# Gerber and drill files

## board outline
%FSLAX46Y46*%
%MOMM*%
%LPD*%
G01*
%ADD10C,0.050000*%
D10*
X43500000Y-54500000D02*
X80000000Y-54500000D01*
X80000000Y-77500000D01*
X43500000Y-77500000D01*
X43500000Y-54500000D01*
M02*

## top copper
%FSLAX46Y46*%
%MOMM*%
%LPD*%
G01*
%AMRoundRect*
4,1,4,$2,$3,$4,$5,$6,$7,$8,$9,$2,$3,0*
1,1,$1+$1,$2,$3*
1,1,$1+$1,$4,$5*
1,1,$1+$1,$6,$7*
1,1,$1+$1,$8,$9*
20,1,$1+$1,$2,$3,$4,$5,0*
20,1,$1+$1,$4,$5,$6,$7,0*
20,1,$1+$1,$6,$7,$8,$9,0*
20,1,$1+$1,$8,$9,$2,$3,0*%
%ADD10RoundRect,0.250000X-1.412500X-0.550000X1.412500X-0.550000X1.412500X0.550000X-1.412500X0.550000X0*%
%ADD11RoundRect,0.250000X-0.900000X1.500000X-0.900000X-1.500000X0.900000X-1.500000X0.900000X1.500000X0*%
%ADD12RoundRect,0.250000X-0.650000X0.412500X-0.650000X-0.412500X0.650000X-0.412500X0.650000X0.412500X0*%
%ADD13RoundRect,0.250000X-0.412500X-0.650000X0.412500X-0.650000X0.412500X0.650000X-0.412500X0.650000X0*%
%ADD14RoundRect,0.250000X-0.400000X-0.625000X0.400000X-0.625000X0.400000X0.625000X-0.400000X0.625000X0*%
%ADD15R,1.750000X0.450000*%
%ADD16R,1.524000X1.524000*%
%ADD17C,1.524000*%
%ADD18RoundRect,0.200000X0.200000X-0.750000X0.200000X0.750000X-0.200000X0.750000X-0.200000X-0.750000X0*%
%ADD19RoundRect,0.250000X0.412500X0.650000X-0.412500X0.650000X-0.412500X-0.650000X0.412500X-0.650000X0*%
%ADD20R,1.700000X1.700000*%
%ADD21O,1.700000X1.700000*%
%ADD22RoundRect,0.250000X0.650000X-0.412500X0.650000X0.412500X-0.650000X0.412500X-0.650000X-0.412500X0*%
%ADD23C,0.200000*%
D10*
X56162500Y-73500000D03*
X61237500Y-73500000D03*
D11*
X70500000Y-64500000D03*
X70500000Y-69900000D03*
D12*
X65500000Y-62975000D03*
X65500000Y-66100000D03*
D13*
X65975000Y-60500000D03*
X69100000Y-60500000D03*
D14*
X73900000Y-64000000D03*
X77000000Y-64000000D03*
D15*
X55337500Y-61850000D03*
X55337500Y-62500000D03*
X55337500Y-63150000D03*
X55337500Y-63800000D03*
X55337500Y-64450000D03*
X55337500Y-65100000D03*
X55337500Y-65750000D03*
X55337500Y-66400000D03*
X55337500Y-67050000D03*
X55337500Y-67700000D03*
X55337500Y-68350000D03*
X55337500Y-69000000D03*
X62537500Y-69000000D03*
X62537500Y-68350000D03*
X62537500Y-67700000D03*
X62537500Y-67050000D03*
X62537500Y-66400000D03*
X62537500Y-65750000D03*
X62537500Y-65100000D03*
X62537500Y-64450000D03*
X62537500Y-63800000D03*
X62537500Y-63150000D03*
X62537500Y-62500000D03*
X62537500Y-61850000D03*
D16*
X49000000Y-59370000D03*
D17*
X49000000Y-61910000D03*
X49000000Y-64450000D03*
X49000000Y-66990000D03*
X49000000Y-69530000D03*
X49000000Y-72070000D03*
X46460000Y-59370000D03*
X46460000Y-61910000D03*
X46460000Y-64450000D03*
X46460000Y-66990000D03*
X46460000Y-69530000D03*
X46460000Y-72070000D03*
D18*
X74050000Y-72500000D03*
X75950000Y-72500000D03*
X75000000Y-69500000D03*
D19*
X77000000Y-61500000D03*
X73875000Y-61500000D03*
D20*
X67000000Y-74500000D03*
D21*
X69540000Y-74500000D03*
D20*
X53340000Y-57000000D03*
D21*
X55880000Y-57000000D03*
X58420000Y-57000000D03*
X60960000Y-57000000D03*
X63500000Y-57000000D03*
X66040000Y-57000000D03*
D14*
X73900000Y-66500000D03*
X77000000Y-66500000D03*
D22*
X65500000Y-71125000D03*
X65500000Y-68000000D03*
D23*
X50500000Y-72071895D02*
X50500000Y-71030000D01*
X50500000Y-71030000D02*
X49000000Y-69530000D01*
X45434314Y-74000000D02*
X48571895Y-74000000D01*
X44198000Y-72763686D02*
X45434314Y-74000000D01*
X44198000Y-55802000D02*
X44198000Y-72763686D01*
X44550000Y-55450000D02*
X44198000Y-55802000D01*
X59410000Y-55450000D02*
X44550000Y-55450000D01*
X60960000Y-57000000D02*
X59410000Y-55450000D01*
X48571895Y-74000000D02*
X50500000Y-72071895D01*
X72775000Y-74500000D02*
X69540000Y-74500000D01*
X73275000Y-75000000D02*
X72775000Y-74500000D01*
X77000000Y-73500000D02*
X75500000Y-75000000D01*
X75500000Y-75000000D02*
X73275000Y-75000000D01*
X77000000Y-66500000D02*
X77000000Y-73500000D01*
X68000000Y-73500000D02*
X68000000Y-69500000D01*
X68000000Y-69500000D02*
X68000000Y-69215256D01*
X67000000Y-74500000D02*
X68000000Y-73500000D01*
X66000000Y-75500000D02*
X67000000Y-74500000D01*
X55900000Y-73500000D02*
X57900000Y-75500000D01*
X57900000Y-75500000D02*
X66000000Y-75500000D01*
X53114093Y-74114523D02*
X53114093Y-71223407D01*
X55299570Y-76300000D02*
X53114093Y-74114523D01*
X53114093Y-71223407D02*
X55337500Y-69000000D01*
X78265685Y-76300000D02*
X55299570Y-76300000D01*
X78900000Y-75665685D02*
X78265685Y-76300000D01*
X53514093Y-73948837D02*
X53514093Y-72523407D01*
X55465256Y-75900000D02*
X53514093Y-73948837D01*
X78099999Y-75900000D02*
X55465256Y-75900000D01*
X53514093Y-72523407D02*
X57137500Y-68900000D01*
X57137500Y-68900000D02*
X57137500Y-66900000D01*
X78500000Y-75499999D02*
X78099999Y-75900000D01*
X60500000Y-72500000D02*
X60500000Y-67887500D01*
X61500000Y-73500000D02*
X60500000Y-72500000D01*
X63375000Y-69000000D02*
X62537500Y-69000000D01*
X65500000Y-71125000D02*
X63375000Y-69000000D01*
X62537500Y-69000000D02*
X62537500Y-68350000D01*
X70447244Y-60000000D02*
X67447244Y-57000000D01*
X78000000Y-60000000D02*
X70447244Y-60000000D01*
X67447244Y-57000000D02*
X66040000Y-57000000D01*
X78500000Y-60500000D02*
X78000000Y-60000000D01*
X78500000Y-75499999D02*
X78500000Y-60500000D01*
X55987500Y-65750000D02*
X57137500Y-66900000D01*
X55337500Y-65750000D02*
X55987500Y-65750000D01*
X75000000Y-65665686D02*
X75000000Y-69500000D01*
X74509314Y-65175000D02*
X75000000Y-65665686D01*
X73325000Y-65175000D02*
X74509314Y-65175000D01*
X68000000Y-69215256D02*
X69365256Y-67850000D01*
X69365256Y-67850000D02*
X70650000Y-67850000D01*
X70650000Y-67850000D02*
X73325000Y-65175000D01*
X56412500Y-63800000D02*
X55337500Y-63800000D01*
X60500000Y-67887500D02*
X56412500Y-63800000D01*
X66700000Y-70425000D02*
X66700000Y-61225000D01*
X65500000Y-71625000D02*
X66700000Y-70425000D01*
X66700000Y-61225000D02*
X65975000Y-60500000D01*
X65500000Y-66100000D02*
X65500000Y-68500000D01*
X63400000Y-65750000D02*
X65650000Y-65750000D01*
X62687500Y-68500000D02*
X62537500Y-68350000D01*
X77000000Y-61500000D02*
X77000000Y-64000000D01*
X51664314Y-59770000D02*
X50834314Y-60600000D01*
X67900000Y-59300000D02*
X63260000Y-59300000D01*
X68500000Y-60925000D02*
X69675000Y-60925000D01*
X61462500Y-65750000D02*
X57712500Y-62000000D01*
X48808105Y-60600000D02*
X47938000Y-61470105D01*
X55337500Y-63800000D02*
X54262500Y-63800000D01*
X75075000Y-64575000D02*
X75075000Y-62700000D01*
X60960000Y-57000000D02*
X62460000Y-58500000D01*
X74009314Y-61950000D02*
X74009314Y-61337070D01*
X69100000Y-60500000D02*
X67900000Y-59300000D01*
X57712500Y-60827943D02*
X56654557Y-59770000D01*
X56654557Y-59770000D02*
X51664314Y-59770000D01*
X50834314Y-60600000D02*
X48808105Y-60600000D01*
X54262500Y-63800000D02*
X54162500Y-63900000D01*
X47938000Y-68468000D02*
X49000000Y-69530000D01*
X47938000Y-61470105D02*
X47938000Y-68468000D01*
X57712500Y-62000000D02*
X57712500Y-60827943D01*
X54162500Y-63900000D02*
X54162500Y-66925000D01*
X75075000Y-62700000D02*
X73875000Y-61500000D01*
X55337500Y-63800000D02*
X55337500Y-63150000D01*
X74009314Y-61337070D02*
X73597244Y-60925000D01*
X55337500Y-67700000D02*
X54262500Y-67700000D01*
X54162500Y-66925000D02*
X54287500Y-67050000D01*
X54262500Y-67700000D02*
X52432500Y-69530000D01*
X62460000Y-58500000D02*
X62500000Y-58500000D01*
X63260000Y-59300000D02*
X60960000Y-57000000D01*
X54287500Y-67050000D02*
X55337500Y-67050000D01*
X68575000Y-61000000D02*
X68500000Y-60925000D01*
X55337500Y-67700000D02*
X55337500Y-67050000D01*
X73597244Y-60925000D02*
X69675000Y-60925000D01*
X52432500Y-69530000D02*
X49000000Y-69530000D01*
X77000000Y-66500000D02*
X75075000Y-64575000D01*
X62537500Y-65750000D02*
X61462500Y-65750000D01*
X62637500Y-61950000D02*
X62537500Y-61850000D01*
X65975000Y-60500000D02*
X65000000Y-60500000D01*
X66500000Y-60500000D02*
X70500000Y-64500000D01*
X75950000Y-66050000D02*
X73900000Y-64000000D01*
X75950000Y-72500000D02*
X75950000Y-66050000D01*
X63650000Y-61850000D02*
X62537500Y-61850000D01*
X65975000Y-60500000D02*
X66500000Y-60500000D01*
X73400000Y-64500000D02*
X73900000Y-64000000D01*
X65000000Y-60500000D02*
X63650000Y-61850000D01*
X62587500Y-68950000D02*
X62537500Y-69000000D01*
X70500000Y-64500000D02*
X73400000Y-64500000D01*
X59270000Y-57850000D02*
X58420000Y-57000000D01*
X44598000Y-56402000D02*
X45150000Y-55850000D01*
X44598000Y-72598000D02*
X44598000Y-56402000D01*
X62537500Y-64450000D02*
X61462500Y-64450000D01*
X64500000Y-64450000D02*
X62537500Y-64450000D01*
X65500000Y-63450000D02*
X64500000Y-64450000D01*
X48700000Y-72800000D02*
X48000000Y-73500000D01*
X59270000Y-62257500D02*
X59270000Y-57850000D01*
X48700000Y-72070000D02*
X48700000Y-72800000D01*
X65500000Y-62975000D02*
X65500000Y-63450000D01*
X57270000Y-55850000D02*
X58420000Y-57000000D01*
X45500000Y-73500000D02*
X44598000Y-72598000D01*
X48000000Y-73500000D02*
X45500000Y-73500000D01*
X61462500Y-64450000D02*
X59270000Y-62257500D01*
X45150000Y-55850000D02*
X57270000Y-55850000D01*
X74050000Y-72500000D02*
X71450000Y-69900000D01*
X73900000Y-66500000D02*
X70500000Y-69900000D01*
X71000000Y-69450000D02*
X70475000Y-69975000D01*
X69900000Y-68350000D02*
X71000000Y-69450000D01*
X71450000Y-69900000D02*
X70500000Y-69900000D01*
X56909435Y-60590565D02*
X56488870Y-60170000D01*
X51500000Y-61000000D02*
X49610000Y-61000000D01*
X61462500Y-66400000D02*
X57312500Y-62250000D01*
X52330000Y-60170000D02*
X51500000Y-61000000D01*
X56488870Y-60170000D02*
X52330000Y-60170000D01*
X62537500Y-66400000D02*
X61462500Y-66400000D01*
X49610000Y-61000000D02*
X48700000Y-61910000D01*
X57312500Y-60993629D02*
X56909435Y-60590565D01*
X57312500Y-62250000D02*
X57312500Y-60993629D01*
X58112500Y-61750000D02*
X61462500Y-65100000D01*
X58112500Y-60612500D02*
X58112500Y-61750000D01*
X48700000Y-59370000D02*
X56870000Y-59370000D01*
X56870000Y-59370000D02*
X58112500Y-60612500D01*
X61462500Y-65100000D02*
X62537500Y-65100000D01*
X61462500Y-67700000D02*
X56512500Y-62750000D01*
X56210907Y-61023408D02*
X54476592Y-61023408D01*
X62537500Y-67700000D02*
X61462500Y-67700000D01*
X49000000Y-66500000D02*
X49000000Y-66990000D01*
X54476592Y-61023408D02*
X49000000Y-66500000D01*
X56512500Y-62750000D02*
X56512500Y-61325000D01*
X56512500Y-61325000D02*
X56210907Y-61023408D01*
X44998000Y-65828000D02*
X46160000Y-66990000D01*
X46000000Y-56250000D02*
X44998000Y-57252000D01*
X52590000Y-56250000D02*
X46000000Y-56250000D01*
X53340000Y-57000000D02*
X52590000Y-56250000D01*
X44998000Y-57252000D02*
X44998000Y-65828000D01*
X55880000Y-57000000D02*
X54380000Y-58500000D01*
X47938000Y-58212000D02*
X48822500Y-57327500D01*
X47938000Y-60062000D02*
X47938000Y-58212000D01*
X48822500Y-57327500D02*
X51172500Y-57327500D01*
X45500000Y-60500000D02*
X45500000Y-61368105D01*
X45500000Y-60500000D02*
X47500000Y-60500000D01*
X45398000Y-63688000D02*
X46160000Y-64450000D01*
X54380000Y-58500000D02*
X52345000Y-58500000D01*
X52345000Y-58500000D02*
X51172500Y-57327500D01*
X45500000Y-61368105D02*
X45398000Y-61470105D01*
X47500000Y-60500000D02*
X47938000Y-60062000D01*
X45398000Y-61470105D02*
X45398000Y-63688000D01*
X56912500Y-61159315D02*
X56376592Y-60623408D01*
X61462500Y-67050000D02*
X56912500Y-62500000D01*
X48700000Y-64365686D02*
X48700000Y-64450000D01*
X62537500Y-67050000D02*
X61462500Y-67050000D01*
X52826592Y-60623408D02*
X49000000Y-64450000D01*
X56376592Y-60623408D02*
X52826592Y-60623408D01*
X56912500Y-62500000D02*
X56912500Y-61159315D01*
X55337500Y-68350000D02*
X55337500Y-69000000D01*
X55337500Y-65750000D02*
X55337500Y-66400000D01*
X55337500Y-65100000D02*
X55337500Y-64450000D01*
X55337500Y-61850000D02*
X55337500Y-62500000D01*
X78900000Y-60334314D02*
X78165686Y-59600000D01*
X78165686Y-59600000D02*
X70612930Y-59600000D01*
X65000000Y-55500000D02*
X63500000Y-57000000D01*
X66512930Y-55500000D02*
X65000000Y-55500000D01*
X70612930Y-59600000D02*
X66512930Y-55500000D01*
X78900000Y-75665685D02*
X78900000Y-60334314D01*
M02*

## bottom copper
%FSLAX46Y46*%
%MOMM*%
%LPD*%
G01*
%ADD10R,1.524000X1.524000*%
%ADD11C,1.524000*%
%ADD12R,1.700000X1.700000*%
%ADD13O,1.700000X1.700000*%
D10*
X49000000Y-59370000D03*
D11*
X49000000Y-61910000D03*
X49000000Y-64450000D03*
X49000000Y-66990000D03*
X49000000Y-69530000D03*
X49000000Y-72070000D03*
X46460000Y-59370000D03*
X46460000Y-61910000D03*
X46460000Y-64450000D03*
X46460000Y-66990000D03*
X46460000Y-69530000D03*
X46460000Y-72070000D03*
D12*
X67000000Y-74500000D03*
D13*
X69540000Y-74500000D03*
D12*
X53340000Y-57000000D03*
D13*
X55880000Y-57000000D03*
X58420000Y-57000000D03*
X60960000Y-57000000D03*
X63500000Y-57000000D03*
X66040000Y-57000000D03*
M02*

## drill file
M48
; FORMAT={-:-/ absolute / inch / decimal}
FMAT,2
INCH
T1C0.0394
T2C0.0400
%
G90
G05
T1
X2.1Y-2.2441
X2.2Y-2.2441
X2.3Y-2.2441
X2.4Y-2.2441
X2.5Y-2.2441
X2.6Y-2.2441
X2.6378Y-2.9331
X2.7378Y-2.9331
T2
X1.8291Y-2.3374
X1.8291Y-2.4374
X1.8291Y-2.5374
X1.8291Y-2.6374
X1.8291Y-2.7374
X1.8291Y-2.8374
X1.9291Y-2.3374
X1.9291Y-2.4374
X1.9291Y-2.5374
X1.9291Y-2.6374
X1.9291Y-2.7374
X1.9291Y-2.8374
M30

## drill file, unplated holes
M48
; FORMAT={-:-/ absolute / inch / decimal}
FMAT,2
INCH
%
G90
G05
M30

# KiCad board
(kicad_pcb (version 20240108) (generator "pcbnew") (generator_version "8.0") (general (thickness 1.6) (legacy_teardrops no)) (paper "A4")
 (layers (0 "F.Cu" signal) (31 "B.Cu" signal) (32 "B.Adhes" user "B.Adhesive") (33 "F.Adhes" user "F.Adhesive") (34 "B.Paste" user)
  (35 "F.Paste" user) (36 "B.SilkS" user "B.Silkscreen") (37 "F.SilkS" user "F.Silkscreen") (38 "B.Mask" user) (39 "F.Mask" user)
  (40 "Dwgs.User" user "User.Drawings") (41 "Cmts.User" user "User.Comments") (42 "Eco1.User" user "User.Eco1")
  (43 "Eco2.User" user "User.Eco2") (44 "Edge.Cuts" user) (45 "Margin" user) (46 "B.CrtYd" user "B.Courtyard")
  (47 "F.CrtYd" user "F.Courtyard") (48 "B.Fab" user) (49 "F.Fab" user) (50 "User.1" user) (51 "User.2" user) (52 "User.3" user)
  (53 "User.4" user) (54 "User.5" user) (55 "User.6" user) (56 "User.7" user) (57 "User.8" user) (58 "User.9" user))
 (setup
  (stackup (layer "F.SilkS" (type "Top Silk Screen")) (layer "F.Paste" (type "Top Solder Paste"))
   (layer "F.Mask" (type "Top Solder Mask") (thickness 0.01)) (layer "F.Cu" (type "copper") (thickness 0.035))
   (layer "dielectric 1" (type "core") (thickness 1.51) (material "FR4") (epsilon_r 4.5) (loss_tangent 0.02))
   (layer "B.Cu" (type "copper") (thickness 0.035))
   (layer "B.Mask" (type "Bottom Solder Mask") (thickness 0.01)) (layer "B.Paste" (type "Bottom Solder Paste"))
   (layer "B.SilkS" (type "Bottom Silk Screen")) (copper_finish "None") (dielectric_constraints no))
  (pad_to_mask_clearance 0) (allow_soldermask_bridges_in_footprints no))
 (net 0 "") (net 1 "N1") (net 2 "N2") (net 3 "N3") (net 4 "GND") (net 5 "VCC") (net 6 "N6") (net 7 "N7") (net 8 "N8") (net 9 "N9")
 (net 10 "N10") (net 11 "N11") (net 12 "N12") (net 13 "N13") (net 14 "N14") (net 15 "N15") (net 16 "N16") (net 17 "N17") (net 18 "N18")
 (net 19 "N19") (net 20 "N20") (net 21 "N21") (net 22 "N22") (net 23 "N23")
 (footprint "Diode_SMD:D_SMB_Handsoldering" (layer "F.Cu") (at 70.5 67.2 -90)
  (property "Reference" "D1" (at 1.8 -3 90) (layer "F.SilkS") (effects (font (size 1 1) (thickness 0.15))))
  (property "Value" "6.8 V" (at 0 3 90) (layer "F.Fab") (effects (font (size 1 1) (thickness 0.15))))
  (pad "1" smd roundrect (at -2.7 0 270) (size 3.5 2.3) (layers "F.Cu" "F.Paste" "F.Mask") (roundrect_rratio 0.1086956522) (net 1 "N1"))
  (pad "2" smd roundrect (at 2.7 0 270) (size 3.5 2.3) (layers "F.Cu" "F.Paste" "F.Mask") (roundrect_rratio 0.1086956522) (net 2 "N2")))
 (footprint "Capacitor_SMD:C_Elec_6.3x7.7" (layer "F.Cu") (at 58.7 73.5)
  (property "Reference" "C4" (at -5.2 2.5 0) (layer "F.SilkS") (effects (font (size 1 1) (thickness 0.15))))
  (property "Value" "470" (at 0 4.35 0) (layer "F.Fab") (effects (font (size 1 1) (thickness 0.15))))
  (pad "1" smd roundrect (at -2.5375 0) (size 3.325 1.6) (layers "F.Cu" "F.Paste" "F.Mask") (roundrect_rratio 0.15625) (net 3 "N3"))
  (pad "2" smd roundrect (at 2.5375 0) (size 3.325 1.6) (layers "F.Cu" "F.Paste" "F.Mask") (roundrect_rratio 0.15625) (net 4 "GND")))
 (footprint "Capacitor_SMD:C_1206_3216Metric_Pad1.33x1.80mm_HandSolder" (layer "F.Cu") (at 65.5 64.5375 -90)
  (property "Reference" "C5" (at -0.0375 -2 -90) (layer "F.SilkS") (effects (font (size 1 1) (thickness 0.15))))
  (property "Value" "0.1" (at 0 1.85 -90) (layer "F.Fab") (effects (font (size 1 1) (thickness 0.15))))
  (pad "1" smd roundrect (at -1.5625 0 270) (size 1.325 1.8) (layers "F.Cu" "F.Paste" "F.Mask") (roundrect_rratio 0.188679) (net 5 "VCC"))
  (pad "2" smd roundrect (at 1.5625 0 270) (size 1.325 1.8) (layers "F.Cu" "F.Paste" "F.Mask") (roundrect_rratio 0.188679) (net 4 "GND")))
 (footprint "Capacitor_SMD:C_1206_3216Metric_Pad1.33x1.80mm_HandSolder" (layer "F.Cu") (at 65.5 69.5625 90)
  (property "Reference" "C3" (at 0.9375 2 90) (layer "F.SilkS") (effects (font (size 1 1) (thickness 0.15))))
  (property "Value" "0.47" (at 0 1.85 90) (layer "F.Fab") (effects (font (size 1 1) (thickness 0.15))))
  (pad "1" smd roundrect (at -1.5625 0 90) (size 1.325 1.8) (layers "F.Cu" "F.Paste" "F.Mask") (roundrect_rratio 0.188679) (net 1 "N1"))
  (pad "2" smd roundrect (at 1.5625 0 90) (size 1.325 1.8) (layers "F.Cu" "F.Paste" "F.Mask") (roundrect_rratio 0.188679) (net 4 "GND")))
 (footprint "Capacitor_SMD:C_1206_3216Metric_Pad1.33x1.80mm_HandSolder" (layer "F.Cu") (at 67.5375 60.5)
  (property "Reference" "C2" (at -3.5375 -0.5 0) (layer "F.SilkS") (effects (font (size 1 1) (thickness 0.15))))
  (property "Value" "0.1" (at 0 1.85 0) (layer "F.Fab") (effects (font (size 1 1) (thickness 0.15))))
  (pad "1" smd roundrect (at -1.5625 0) (size 1.325 1.8) (layers "F.Cu" "F.Paste" "F.Mask") (roundrect_rratio 0.188679) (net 1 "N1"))
  (pad "2" smd roundrect (at 1.5625 0) (size 1.325 1.8) (layers "F.Cu" "F.Paste" "F.Mask") (roundrect_rratio 0.188679) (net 4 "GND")))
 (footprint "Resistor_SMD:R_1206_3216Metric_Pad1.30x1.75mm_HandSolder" (layer "F.Cu") (at 75.45 64)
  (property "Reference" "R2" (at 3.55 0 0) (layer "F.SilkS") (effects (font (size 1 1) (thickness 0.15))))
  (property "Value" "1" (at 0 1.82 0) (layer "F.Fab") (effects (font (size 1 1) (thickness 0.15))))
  (pad "1" smd roundrect (at -1.55 0) (size 1.3 1.75) (layers "F.Cu" "F.Paste" "F.Mask") (roundrect_rratio 0.192308) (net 1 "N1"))
  (pad "2" smd roundrect (at 1.55 0) (size 1.3 1.75) (layers "F.Cu" "F.Paste" "F.Mask") (roundrect_rratio 0.192308) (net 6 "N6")))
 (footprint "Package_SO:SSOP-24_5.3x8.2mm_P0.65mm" (layer "F.Cu") (at 58.9375 65.425)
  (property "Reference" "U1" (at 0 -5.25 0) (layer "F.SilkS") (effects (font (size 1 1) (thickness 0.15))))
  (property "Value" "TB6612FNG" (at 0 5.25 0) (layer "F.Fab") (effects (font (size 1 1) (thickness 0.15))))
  (pad "1" smd rect (at -3.6 -3.575) (size 1.75 0.45) (layers "F.Cu" "F.Paste" "F.Mask") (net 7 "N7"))
  (pad "2" smd rect (at -3.6 -2.925) (size 1.75 0.45) (layers "F.Cu" "F.Paste" "F.Mask") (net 7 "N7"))
  (pad "3" smd rect (at -3.6 -2.275) (size 1.75 0.45) (layers "F.Cu" "F.Paste" "F.Mask") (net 4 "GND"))
  (pad "4" smd rect (at -3.6 -1.625) (size 1.75 0.45) (layers "F.Cu" "F.Paste" "F.Mask") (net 4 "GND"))
  (pad "5" smd rect (at -3.6 -0.975) (size 1.75 0.45) (layers "F.Cu" "F.Paste" "F.Mask") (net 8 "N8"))
  (pad "6" smd rect (at -3.6 -0.325) (size 1.75 0.45) (layers "F.Cu" "F.Paste" "F.Mask") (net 8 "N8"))
  (pad "7" smd rect (at -3.6 0.325) (size 1.75 0.45) (layers "F.Cu" "F.Paste" "F.Mask") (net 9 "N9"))
  (pad "8" smd rect (at -3.6 0.975) (size 1.75 0.45) (layers "F.Cu" "F.Paste" "F.Mask") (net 9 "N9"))
  (pad "9" smd rect (at -3.6 1.625) (size 1.75 0.45) (layers "F.Cu" "F.Paste" "F.Mask") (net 4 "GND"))
  (pad "10" smd rect (at -3.6 2.275) (size 1.75 0.45) (layers "F.Cu" "F.Paste" "F.Mask") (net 4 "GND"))
  (pad "11" smd rect (at -3.6 2.925) (size 1.75 0.45) (layers "F.Cu" "F.Paste" "F.Mask") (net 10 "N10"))
  (pad "12" smd rect (at -3.6 3.575) (size 1.75 0.45) (layers "F.Cu" "F.Paste" "F.Mask") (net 10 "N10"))
  (pad "13" smd rect (at 3.6 3.575) (size 1.75 0.45) (layers "F.Cu" "F.Paste" "F.Mask") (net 1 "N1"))
  (pad "14" smd rect (at 3.6 2.925) (size 1.75 0.45) (layers "F.Cu" "F.Paste" "F.Mask") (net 1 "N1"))
  (pad "15" smd rect (at 3.6 2.275) (size 1.75 0.45) (layers "F.Cu" "F.Paste" "F.Mask") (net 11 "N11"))
  (pad "16" smd rect (at 3.6 1.625) (size 1.75 0.45) (layers "F.Cu" "F.Paste" "F.Mask") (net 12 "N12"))
  (pad "17" smd rect (at 3.6 0.975) (size 1.75 0.45) (layers "F.Cu" "F.Paste" "F.Mask") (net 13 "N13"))
  (pad "18" smd rect (at 3.6 0.325) (size 1.75 0.45) (layers "F.Cu" "F.Paste" "F.Mask") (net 4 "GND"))
  (pad "19" smd rect (at 3.6 -0.325) (size 1.75 0.45) (layers "F.Cu" "F.Paste" "F.Mask") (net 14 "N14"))
  (pad "20" smd rect (at 3.6 -0.975) (size 1.75 0.45) (layers "F.Cu" "F.Paste" "F.Mask") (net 5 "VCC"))
  (pad "21" smd rect (at 3.6 -1.625) (size 1.75 0.45) (layers "F.Cu" "F.Paste" "F.Mask") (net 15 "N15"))
  (pad "22" smd rect (at 3.6 -2.275) (size 1.75 0.45) (layers "F.Cu" "F.Paste" "F.Mask") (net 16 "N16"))
  (pad "23" smd rect (at 3.6 -2.925) (size 1.75 0.45) (layers "F.Cu" "F.Paste" "F.Mask") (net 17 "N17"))
  (pad "24" smd rect (at 3.6 -3.575) (size 1.75 0.45) (layers "F.Cu" "F.Paste" "F.Mask") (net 1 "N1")))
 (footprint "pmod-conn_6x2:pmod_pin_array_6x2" (layer "F.Cu") (at 47.73 65.72)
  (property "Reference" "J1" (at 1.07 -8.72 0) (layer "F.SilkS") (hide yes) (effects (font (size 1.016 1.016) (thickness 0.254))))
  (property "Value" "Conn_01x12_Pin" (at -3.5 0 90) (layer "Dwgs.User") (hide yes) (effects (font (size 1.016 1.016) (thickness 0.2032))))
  (pad "1" thru_hole rect (at 1.27 -6.35) (size 1.524 1.524) (drill 1.016) (layers "*.Cu" "*.Mask" "F.SilkS") (remove_unused_layers no)
   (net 14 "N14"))
  (pad "2" thru_hole circle (at 1.27 -3.81 270) (size 1.524 1.524) (drill 1.016) (layers "*.Cu" "*.Mask" "F.SilkS")
   (remove_unused_layers no) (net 13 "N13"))
  (pad "3" thru_hole circle (at 1.27 -1.27 270) (size 1.524 1.524) (drill 1.016) (layers "*.Cu" "*.Mask" "F.SilkS")
   (remove_unused_layers no) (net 12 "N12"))
  (pad "4" thru_hole circle (at 1.27 1.27 270) (size 1.524 1.524) (drill 1.016) (layers "*.Cu" "*.Mask" "F.SilkS") (remove_unused_layers no)
   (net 11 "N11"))
  (pad "5" thru_hole circle (at 1.27 3.81 270) (size 1.524 1.524) (drill 1.016) (layers "*.Cu" "*.Mask" "F.SilkS") (remove_unused_layers no)
   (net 4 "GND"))
  (pad "6" thru_hole circle (at 1.27 6.35 270) (size 1.524 1.524) (drill 1.016) (layers "*.Cu" "*.Mask" "F.SilkS") (remove_unused_layers no)
   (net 5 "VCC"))
  (pad "7" thru_hole circle (at -1.27 -6.35 270) (size 1.524 1.524) (drill 1.016) (layers "*.Cu" "*.Mask" "F.SilkS")
   (remove_unused_layers no) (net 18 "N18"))
  (pad "8" thru_hole circle (at -1.27 -3.81 270) (size 1.524 1.524) (drill 1.016) (layers "*.Cu" "*.Mask" "F.SilkS")
   (remove_unused_layers no) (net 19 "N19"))
  (pad "9" thru_hole circle (at -1.27 -1.27 270) (size 1.524 1.524) (drill 1.016) (layers "*.Cu" "*.Mask" "F.SilkS")
   (remove_unused_layers no) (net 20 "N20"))
  (pad "10" thru_hole circle (at -1.27 1.27 270) (size 1.524 1.524) (drill 1.016) (layers "*.Cu" "*.Mask" "F.SilkS")
   (remove_unused_layers no) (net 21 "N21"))
  (pad "11" thru_hole circle (at -1.27 3.81 270) (size 1.524 1.524) (drill 1.016) (layers "*.Cu" "*.Mask" "F.SilkS")
   (remove_unused_layers no) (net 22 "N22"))
  (pad "12" thru_hole circle (at -1.27 6.35 270) (size 1.524 1.524) (drill 1.016) (layers "*.Cu" "*.Mask" "F.SilkS")
   (remove_unused_layers no) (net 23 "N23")))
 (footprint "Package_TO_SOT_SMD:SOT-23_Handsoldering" (layer "F.Cu") (at 75 71 90)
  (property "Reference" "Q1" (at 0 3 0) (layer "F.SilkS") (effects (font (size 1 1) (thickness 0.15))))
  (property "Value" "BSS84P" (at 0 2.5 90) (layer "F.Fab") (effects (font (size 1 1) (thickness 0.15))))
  (pad "1" smd roundrect (at -1.5 -0.95 90) (size 1.9 0.8) (layers "F.Cu" "F.Paste" "F.Mask") (roundrect_rratio 0.25) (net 2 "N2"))
  (pad "2" smd roundrect (at -1.5 0.95 90) (size 1.9 0.8) (layers "F.Cu" "F.Paste" "F.Mask") (roundrect_rratio 0.25) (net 1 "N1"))
  (pad "3" smd roundrect (at 1.5 0 90) (size 1.9 0.8) (layers "F.Cu" "F.Paste" "F.Mask") (roundrect_rratio 0.25) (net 3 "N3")))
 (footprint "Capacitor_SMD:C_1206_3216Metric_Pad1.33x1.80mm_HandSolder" (layer "F.Cu") (at 75.4375 61.5 180)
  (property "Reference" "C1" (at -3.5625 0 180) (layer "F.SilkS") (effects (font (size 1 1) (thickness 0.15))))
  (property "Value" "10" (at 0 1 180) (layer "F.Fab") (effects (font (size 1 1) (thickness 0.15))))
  (pad "1" smd roundrect (at -1.5625 0 180) (size 1.325 1.8) (layers "F.Cu" "F.Paste" "F.Mask") (roundrect_rratio 0.188679) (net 6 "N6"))
  (pad "2" smd roundrect (at 1.5625 0 180) (size 1.325 1.8) (layers "F.Cu" "F.Paste" "F.Mask") (roundrect_rratio 0.188679) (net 4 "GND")))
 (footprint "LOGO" (layer "F.Cu") (at 75.5 57.5)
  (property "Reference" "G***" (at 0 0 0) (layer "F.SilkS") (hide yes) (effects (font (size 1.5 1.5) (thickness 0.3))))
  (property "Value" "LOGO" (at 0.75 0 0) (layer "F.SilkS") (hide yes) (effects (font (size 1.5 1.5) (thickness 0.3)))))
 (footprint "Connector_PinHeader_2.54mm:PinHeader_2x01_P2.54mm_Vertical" (layer "F.Cu") (at 67 74.5)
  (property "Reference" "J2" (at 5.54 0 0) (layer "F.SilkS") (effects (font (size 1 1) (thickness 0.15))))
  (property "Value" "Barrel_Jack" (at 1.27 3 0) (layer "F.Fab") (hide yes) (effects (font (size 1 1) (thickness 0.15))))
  (pad "1" thru_hole rect (at 0 0) (size 1.7 1.7) (drill 1) (layers "*.Cu" "*.Mask") (remove_unused_layers no) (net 3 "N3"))
  (pad "2" thru_hole oval (at 2.54 0) (size 1.7 1.7) (drill 1) (layers "*.Cu" "*.Mask") (remove_unused_layers no) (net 4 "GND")))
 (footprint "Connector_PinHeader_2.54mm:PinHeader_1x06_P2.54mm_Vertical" (layer "F.Cu") (at 53.34 57 90)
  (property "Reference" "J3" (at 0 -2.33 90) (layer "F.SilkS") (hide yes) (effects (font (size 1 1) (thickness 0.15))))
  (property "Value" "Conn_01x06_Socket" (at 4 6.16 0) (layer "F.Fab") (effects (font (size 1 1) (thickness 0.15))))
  (pad "1" thru_hole rect (at 0 0 90) (size 1.7 1.7) (drill 1) (layers "*.Cu" "*.Mask") (remove_unused_layers no) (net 21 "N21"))
  (pad "2" thru_hole oval (at 0 2.54 90) (size 1.7 1.7) (drill 1) (layers "*.Cu" "*.Mask") (remove_unused_layers no) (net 20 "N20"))
  (pad "3" thru_hole oval (at 0 5.08 90) (size 1.7 1.7) (drill 1) (layers "*.Cu" "*.Mask") (remove_unused_layers no) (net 5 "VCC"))
  (pad "4" thru_hole oval (at 0 7.62 90) (size 1.7 1.7) (drill 1) (layers "*.Cu" "*.Mask") (remove_unused_layers no) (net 4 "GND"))
  (pad "5" thru_hole oval (at 0 10.16 90) (size 1.7 1.7) (drill 1) (layers "*.Cu" "*.Mask") (remove_unused_layers no) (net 10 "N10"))
  (pad "6" thru_hole oval (at 0 12.7 90) (size 1.7 1.7) (drill 1) (layers "*.Cu" "*.Mask") (remove_unused_layers no) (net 9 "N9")))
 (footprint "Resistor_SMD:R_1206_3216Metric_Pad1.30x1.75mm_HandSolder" (layer "F.Cu") (at 75.45 66.5)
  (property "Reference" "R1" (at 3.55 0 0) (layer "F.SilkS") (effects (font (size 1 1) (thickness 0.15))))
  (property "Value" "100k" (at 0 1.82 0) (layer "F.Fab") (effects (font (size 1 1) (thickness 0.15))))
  (pad "1" smd roundrect (at -1.55 0) (size 1.3 1.75) (layers "F.Cu" "F.Paste" "F.Mask") (roundrect_rratio 0.192308) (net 2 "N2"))
  (pad "2" smd roundrect (at 1.55 0) (size 1.3 1.75) (layers "F.Cu" "F.Paste" "F.Mask") (roundrect_rratio 0.192308) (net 4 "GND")))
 (gr_rect (start 43.5 54.5) (end 80 77.5) (stroke (width 0.05) (type default)) (fill none) (layer "Edge.Cuts"))
 (segment (start 77 61.5) (end 77 64) (width 0.2) (layer "F.Cu") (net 6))
 (segment (start 60.5 67.8875) (end 56.4125 63.8) (width 0.2) (layer "F.Cu") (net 4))
 (segment (start 51.664314 59.77) (end 50.834314 60.6) (width 0.2) (layer "F.Cu") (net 4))
 (segment (start 67.9 59.3) (end 63.26 59.3) (width 0.2) (layer "F.Cu") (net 4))
 (segment (start 60.96 57) (end 59.41 55.45) (width 0.2) (layer "F.Cu") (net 4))
 (segment (start 68.5 60.925) (end 69.675 60.925) (width 0.2) (layer "F.Cu") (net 4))
 (segment (start 63.4 65.75) (end 65.65 65.75) (width 0.2) (layer "F.Cu") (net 4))
 (segment (start 61.4625 65.75) (end 57.7125 62) (width 0.2) (layer "F.Cu") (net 4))
 (segment (start 65.5 66.1) (end 65.5 68.5) (width 0.2) (layer "F.Cu") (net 4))
 (segment (start 48.808105 60.6) (end 47.938 61.470105) (width 0.2) (layer "F.Cu") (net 4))
 (segment (start 55.3375 63.8) (end 54.2625 63.8) (width 0.2) (layer "F.Cu") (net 4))
 (segment (start 75.075 64.575) (end 75.075 62.7) (width 0.2) (layer "F.Cu") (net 4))
 (segment (start 60.96 57) (end 62.46 58.5) (width 0.2) (layer "F.Cu") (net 4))
 (segment (start 74.009314 61.95) (end 74.009314 61.33707) (width 0.2) (layer "F.Cu") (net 4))
 (segment (start 77 73.5) (end 75.5 75) (width 0.2) (layer "F.Cu") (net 4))
 (segment (start 45.434314 74) (end 48.571895 74) (width 0.2) (layer "F.Cu") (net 4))
 (segment (start 44.198 55.802) (end 44.198 72.763686) (width 0.2) (layer "F.Cu") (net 4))
 (segment (start 69.1 60.5) (end 67.9 59.3) (width 0.2) (layer "F.Cu") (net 4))
 (segment (start 57.7125 60.827943) (end 56.654557 59.77) (width 0.2) (layer "F.Cu") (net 4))
 (segment (start 59.41 55.45) (end 44.55 55.45) (width 0.2) (layer "F.Cu") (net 4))
 (segment (start 56.654557 59.77) (end 51.664314 59.77) (width 0.2) (layer "F.Cu") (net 4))
 (segment (start 72.775 74.5) (end 69.54 74.5) (width 0.2) (layer "F.Cu") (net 4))
 (segment (start 50.834314 60.6) (end 48.808105 60.6) (width 0.2) (layer "F.Cu") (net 4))
 (segment (start 54.2625 63.8) (end 54.1625 63.9) (width 0.2) (layer "F.Cu") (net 4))
 (segment (start 47.938 68.468) (end 49 69.53) (width 0.2) (layer "F.Cu") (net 4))
 (segment (start 48.571895 74) (end 50.5 72.071895) (width 0.2) (layer "F.Cu") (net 4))
 (segment (start 47.938 61.470105) (end 47.938 68.468) (width 0.2) (layer "F.Cu") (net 4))
 (segment (start 57.7125 62) (end 57.7125 60.827943) (width 0.2) (layer "F.Cu") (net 4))
 (segment (start 75.5 75) (end 73.275 75) (width 0.2) (layer "F.Cu") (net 4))
 (segment (start 56.4125 63.8) (end 55.3375 63.8) (width 0.2) (layer "F.Cu") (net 4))
 (segment (start 54.1625 63.9) (end 54.1625 66.925) (width 0.2) (layer "F.Cu") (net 4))
 (segment (start 73.275 75) (end 72.775 74.5) (width 0.2) (layer "F.Cu") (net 4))
 (segment (start 75.075 62.7) (end 73.875 61.5) (width 0.2) (layer "F.Cu") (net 4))
 (segment (start 44.55 55.45) (end 44.198 55.802) (width 0.2) (layer "F.Cu") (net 4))
 (segment (start 55.3375 63.8) (end 55.3375 63.15) (width 0.2) (layer "F.Cu") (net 4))
 (segment (start 50.5 72.071895) (end 50.5 71.03) (width 0.2) (layer "F.Cu") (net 4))
 (segment (start 74.009314 61.33707) (end 73.597244 60.925) (width 0.2) (layer "F.Cu") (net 4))
 (segment (start 61.5 73.5) (end 60.5 72.5) (width 0.2) (layer "F.Cu") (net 4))
 (segment (start 55.3375 67.7) (end 54.2625 67.7) (width 0.2) (layer "F.Cu") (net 4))
 (segment (start 54.1625 66.925) (end 54.2875 67.05) (width 0.2) (layer "F.Cu") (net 4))
 (segment (start 50.5 71.03) (end 49 69.53) (width 0.2) (layer "F.Cu") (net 4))
 (segment (start 44.198 72.763686) (end 45.434314 74) (width 0.2) (layer "F.Cu") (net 4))
 (segment (start 54.2625 67.7) (end 52.4325 69.53) (width 0.2) (layer "F.Cu") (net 4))
 (segment (start 62.46 58.5) (end 62.5 58.5) (width 0.2) (layer "F.Cu") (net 4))
 (segment (start 63.26 59.3) (end 60.96 57) (width 0.2) (layer "F.Cu") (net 4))
 (segment (start 54.2875 67.05) (end 55.3375 67.05) (width 0.2) (layer "F.Cu") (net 4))
 (segment (start 68.575 61) (end 68.5 60.925) (width 0.2) (layer "F.Cu") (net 4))
 (segment (start 55.3375 67.7) (end 55.3375 67.05) (width 0.2) (layer "F.Cu") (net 4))
 (segment (start 73.597244 60.925) (end 69.675 60.925) (width 0.2) (layer "F.Cu") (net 4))
 (segment (start 60.5 72.5) (end 60.5 67.8875) (width 0.2) (layer "F.Cu") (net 4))
 (segment (start 77 66.5) (end 77 73.5) (width 0.2) (layer "F.Cu") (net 4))
 (segment (start 52.4325 69.53) (end 49 69.53) (width 0.2) (layer "F.Cu") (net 4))
 (segment (start 77 66.5) (end 75.075 64.575) (width 0.2) (layer "F.Cu") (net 4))
 (segment (start 62.5375 65.75) (end 61.4625 65.75) (width 0.2) (layer "F.Cu") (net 4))
 (segment (start 62.6375 61.95) (end 62.5375 61.85) (width 0.2) (layer "F.Cu") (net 1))
 (segment (start 65.975 60.5) (end 65 60.5) (width 0.2) (layer "F.Cu") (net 1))
 (segment (start 62.6875 68.5) (end 62.5375 68.35) (width 0.2) (layer "F.Cu") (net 1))
 (segment (start 66.5 60.5) (end 70.5 64.5) (width 0.2) (layer "F.Cu") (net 1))
 (segment (start 75.95 66.05) (end 73.9 64) (width 0.2) (layer "F.Cu") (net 1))
 (segment (start 66.7 61.225) (end 65.975 60.5) (width 0.2) (layer "F.Cu") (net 1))
 (segment (start 75.95 72.5) (end 75.95 66.05) (width 0.2) (layer "F.Cu") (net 1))
 (segment (start 63.375 69) (end 62.5375 69) (width 0.2) (layer "F.Cu") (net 1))
 (segment (start 62.5375 69) (end 62.5375 68.35) (width 0.2) (layer "F.Cu") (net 1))
 (segment (start 63.65 61.85) (end 62.5375 61.85) (width 0.2) (layer "F.Cu") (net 1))
 (segment (start 65.975 60.5) (end 66.5 60.5) (width 0.2) (layer "F.Cu") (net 1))
 (segment (start 65.5 71.625) (end 66.7 70.425) (width 0.2) (layer "F.Cu") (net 1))
 (segment (start 73.4 64.5) (end 73.9 64) (width 0.2) (layer "F.Cu") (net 1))
 (segment (start 66.7 70.425) (end 66.7 61.225) (width 0.2) (layer "F.Cu") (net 1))
 (segment (start 65 60.5) (end 63.65 61.85) (width 0.2) (layer "F.Cu") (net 1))
 (segment (start 65.5 71.125) (end 63.375 69) (width 0.2) (layer "F.Cu") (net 1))
 (segment (start 62.5875 68.95) (end 62.5375 69) (width 0.2) (layer "F.Cu") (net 1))
 (segment (start 70.5 64.5) (end 73.4 64.5) (width 0.2) (layer "F.Cu") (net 1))
 (segment (start 57.9 75.5) (end 66 75.5) (width 0.2) (layer "F.Cu") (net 3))
 (segment (start 67 74.5) (end 68 73.5) (width 0.2) (layer "F.Cu") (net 3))
 (segment (start 69.365256 67.85) (end 70.65 67.85) (width 0.2) (layer "F.Cu") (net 3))
 (segment (start 66 75.5) (end 67 74.5) (width 0.2) (layer "F.Cu") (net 3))
 (segment (start 70.65 67.85) (end 73.325 65.175) (width 0.2) (layer "F.Cu") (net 3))
 (segment (start 74.509314 65.175) (end 75 65.665686) (width 0.2) (layer "F.Cu") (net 3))
 (segment (start 68 69.5) (end 68 69.215256) (width 0.2) (layer "F.Cu") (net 3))
 (segment (start 55.9 73.5) (end 57.9 75.5) (width 0.2) (layer "F.Cu") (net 3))
 (segment (start 73.325 65.175) (end 74.509314 65.175) (width 0.2) (layer "F.Cu") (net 3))
 (segment (start 68 69.215256) (end 69.365256 67.85) (width 0.2) (layer "F.Cu") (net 3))
 (segment (start 68 73.5) (end 68 69.5) (width 0.2) (layer "F.Cu") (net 3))
 (segment (start 75 65.665686) (end 75 69.5) (width 0.2) (layer "F.Cu") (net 3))
 (segment (start 59.27 57.85) (end 58.42 57) (width 0.2) (layer "F.Cu") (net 5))
 (segment (start 44.598 56.402) (end 45.15 55.85) (width 0.2) (layer "F.Cu") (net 5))
 (segment (start 44.598 72.598) (end 44.598 56.402) (width 0.2) (layer "F.Cu") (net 5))
 (segment (start 62.5375 64.45) (end 61.4625 64.45) (width 0.2) (layer "F.Cu") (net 5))
 (segment (start 64.5 64.45) (end 62.5375 64.45) (width 0.2) (layer "F.Cu") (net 5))
 (segment (start 65.5 63.45) (end 64.5 64.45) (width 0.2) (layer "F.Cu") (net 5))
 (segment (start 48.7 72.8) (end 48 73.5) (width 0.2) (layer "F.Cu") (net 5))
 (segment (start 59.27 62.2575) (end 59.27 57.85) (width 0.2) (layer "F.Cu") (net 5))
 (segment (start 48.7 72.07) (end 48.7 72.8) (width 0.2) (layer "F.Cu") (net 5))
 (segment (start 65.5 62.975) (end 65.5 63.45) (width 0.2) (layer "F.Cu") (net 5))
 (segment (start 57.27 55.85) (end 58.42 57) (width 0.2) (layer "F.Cu") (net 5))
 (segment (start 45.5 73.5) (end 44.598 72.598) (width 0.2) (layer "F.Cu") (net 5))
 (segment (start 48 73.5) (end 45.5 73.5) (width 0.2) (layer "F.Cu") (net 5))
 (segment (start 61.4625 64.45) (end 59.27 62.2575) (width 0.2) (layer "F.Cu") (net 5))
 (segment (start 45.15 55.85) (end 57.27 55.85) (width 0.2) (layer "F.Cu") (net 5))
 (segment (start 74.05 72.5) (end 71.45 69.9) (width 0.2) (layer "F.Cu") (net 2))
 (segment (start 73.9 66.5) (end 70.5 69.9) (width 0.2) (layer "F.Cu") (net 2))
 (segment (start 71 69.45) (end 70.475 69.975) (width 0.2) (layer "F.Cu") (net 2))
 (segment (start 69.9 68.35) (end 71 69.45) (width 0.2) (layer "F.Cu") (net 2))
 (segment (start 71.45 69.9) (end 70.5 69.9) (width 0.2) (layer "F.Cu") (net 2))
 (segment (start 56.909435 60.590565) (end 56.48887 60.17) (width 0.2) (layer "F.Cu") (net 13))
 (segment (start 51.5 61) (end 49.61 61) (width 0.2) (layer "F.Cu") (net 13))
 (segment (start 61.4625 66.4) (end 57.3125 62.25) (width 0.2) (layer "F.Cu") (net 13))
 (segment (start 52.33 60.17) (end 51.5 61) (width 0.2) (layer "F.Cu") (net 13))
 (segment (start 56.48887 60.17) (end 52.33 60.17) (width 0.2) (layer "F.Cu") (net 13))
 (segment (start 62.5375 66.4) (end 61.4625 66.4) (width 0.2) (layer "F.Cu") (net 13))
 (segment (start 49.61 61) (end 48.7 61.91) (width 0.2) (layer "F.Cu") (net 13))
 (segment (start 57.3125 60.993629) (end 56.909435 60.590565) (width 0.2) (layer "F.Cu") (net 13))
 (segment (start 57.3125 62.25) (end 57.3125 60.993629) (width 0.2) (layer "F.Cu") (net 13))
 (segment (start 58.1125 61.75) (end 61.4625 65.1) (width 0.2) (layer "F.Cu") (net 14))
 (segment (start 58.1125 60.6125) (end 58.1125 61.75) (width 0.2) (layer "F.Cu") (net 14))
 (segment (start 48.7 59.37) (end 56.87 59.37) (width 0.2) (layer "F.Cu") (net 14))
 (segment (start 56.87 59.37) (end 58.1125 60.6125) (width 0.2) (layer "F.Cu") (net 14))
 (segment (start 61.4625 65.1) (end 62.5375 65.1) (width 0.2) (layer "F.Cu") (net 14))
 (segment (start 61.4625 67.7) (end 56.5125 62.75) (width 0.2) (layer "F.Cu") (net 11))
 (segment (start 56.210907 61.023408) (end 54.476592 61.023408) (width 0.2) (layer "F.Cu") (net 11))
 (segment (start 62.5375 67.7) (end 61.4625 67.7) (width 0.2) (layer "F.Cu") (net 11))
 (segment (start 49 66.5) (end 49 66.99) (width 0.2) (layer "F.Cu") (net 11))
 (segment (start 54.476592 61.023408) (end 49 66.5) (width 0.2) (layer "F.Cu") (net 11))
 (segment (start 56.5125 62.75) (end 56.5125 61.325) (width 0.2) (layer "F.Cu") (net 11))
 (segment (start 56.5125 61.325) (end 56.210907 61.023408) (width 0.2) (layer "F.Cu") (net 11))
 (segment (start 44.998 65.828) (end 46.16 66.99) (width 0.2) (layer "F.Cu") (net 21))
 (segment (start 46 56.25) (end 44.998 57.252) (width 0.2) (layer "F.Cu") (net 21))
 (segment (start 52.59 56.25) (end 46 56.25) (width 0.2) (layer "F.Cu") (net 21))
 (segment (start 53.34 57) (end 52.59 56.25) (width 0.2) (layer "F.Cu") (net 21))
 (segment (start 44.998 57.252) (end 44.998 65.828) (width 0.2) (layer "F.Cu") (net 21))
 (segment (start 55.88 57) (end 54.38 58.5) (width 0.2) (layer "F.Cu") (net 20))
 (segment (start 47.938 58.212) (end 48.8225 57.3275) (width 0.2) (layer "F.Cu") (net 20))
 (segment (start 47.938 60.062) (end 47.938 58.212) (width 0.2) (layer "F.Cu") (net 20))
 (segment (start 48.8225 57.3275) (end 51.1725 57.3275) (width 0.2) (layer "F.Cu") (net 20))
 (segment (start 45.5 60.5) (end 45.5 61.368105) (width 0.2) (layer "F.Cu") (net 20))
 (segment (start 45.5 60.5) (end 47.5 60.5) (width 0.2) (layer "F.Cu") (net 20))
 (segment (start 45.398 63.688) (end 46.16 64.45) (width 0.2) (layer "F.Cu") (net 20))
 (segment (start 54.38 58.5) (end 52.345 58.5) (width 0.2) (layer "F.Cu") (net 20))
 (segment (start 52.345 58.5) (end 51.1725 57.3275) (width 0.2) (layer "F.Cu") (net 20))
 (segment (start 45.5 61.368105) (end 45.398 61.470105) (width 0.2) (layer "F.Cu") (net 20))
 (segment (start 47.5 60.5) (end 47.938 60.062) (width 0.2) (layer "F.Cu") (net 20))
 (segment (start 45.398 61.470105) (end 45.398 63.688) (width 0.2) (layer "F.Cu") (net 20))
 (segment (start 56.9125 61.159315) (end 56.376592 60.623408) (width 0.2) (layer "F.Cu") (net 12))
 (segment (start 61.4625 67.05) (end 56.9125 62.5) (width 0.2) (layer "F.Cu") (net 12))
 (segment (start 48.7 64.365686) (end 48.7 64.45) (width 0.2) (layer "F.Cu") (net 12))
 (segment (start 62.5375 67.05) (end 61.4625 67.05) (width 0.2) (layer "F.Cu") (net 12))
 (segment (start 52.826592 60.623408) (end 49 64.45) (width 0.2) (layer "F.Cu") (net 12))
 (segment (start 56.376592 60.623408) (end 52.826592 60.623408) (width 0.2) (layer "F.Cu") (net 12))
 (segment (start 56.9125 62.5) (end 56.9125 61.159315) (width 0.2) (layer "F.Cu") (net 12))
 (segment (start 78.165686 59.6) (end 70.61293 59.6) (width 0.2) (layer "F.Cu") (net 10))
 (segment (start 55.3375 68.35) (end 55.3375 69) (width 0.2) (layer "F.Cu") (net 10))
 (segment (start 55.29957 76.3) (end 53.114093 74.114523) (width 0.2) (layer "F.Cu") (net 10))
 (segment (start 78.265685 76.3) (end 55.29957 76.3) (width 0.2) (layer "F.Cu") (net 10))
 (segment (start 78.9 75.665685) (end 78.9 60.334314) (width 0.2) (layer "F.Cu") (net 10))
 (segment (start 53.114093 71.223407) (end 55.3375 69) (width 0.2) (layer "F.Cu") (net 10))
 (segment (start 78.9 60.334314) (end 78.165686 59.6) (width 0.2) (layer "F.Cu") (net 10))
 (segment (start 53.114093 74.114523) (end 53.114093 71.223407) (width 0.2) (layer "F.Cu") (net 10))
 (segment (start 66.51293 55.5) (end 65 55.5) (width 0.2) (layer "F.Cu") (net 10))
 (segment (start 78.9 75.665685) (end 78.265685 76.3) (width 0.2) (layer "F.Cu") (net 10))
 (segment (start 65 55.5) (end 63.5 57) (width 0.2) (layer "F.Cu") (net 10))
 (segment (start 70.61293 59.6) (end 66.51293 55.5) (width 0.2) (layer "F.Cu") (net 10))
 (segment (start 78.099999 75.9) (end 55.465256 75.9) (width 0.2) (layer "F.Cu") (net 9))
 (segment (start 57.1375 68.9) (end 57.1375 66.9) (width 0.2) (layer "F.Cu") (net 9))
 (segment (start 53.514093 72.523407) (end 57.1375 68.9) (width 0.2) (layer "F.Cu") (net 9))
 (segment (start 67.447244 57) (end 66.04 57) (width 0.2) (layer "F.Cu") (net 9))
 (segment (start 70.447244 60) (end 67.447244 57) (width 0.2) (layer "F.Cu") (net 9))
 (segment (start 55.465256 75.9) (end 53.514093 73.948837) (width 0.2) (layer "F.Cu") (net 9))
 (segment (start 78.5 75.499999) (end 78.5 60.5) (width 0.2) (layer "F.Cu") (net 9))
 (segment (start 55.9875 65.75) (end 57.1375 66.9) (width 0.2) (layer "F.Cu") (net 9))
 (segment (start 55.3375 65.75) (end 55.9875 65.75) (width 0.2) (layer "F.Cu") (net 9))
 (segment (start 53.514093 73.948837) (end 53.514093 72.523407) (width 0.2) (layer "F.Cu") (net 9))
 (segment (start 55.3375 65.75) (end 55.3375 66.4) (width 0.2) (layer "F.Cu") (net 9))
 (segment (start 78 60) (end 70.447244 60) (width 0.2) (layer "F.Cu") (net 9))
 (segment (start 78.5 75.499999) (end 78.099999 75.9) (width 0.2) (layer "F.Cu") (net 9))
 (segment (start 78.5 60.5) (end 78 60) (width 0.2) (layer "F.Cu") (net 9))
 (segment (start 55.3375 65.1) (end 55.3375 64.45) (width 0.2) (layer "F.Cu") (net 8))
 (segment (start 55.3375 61.85) (end 55.3375 62.5) (width 0.2) (layer "F.Cu") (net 7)))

